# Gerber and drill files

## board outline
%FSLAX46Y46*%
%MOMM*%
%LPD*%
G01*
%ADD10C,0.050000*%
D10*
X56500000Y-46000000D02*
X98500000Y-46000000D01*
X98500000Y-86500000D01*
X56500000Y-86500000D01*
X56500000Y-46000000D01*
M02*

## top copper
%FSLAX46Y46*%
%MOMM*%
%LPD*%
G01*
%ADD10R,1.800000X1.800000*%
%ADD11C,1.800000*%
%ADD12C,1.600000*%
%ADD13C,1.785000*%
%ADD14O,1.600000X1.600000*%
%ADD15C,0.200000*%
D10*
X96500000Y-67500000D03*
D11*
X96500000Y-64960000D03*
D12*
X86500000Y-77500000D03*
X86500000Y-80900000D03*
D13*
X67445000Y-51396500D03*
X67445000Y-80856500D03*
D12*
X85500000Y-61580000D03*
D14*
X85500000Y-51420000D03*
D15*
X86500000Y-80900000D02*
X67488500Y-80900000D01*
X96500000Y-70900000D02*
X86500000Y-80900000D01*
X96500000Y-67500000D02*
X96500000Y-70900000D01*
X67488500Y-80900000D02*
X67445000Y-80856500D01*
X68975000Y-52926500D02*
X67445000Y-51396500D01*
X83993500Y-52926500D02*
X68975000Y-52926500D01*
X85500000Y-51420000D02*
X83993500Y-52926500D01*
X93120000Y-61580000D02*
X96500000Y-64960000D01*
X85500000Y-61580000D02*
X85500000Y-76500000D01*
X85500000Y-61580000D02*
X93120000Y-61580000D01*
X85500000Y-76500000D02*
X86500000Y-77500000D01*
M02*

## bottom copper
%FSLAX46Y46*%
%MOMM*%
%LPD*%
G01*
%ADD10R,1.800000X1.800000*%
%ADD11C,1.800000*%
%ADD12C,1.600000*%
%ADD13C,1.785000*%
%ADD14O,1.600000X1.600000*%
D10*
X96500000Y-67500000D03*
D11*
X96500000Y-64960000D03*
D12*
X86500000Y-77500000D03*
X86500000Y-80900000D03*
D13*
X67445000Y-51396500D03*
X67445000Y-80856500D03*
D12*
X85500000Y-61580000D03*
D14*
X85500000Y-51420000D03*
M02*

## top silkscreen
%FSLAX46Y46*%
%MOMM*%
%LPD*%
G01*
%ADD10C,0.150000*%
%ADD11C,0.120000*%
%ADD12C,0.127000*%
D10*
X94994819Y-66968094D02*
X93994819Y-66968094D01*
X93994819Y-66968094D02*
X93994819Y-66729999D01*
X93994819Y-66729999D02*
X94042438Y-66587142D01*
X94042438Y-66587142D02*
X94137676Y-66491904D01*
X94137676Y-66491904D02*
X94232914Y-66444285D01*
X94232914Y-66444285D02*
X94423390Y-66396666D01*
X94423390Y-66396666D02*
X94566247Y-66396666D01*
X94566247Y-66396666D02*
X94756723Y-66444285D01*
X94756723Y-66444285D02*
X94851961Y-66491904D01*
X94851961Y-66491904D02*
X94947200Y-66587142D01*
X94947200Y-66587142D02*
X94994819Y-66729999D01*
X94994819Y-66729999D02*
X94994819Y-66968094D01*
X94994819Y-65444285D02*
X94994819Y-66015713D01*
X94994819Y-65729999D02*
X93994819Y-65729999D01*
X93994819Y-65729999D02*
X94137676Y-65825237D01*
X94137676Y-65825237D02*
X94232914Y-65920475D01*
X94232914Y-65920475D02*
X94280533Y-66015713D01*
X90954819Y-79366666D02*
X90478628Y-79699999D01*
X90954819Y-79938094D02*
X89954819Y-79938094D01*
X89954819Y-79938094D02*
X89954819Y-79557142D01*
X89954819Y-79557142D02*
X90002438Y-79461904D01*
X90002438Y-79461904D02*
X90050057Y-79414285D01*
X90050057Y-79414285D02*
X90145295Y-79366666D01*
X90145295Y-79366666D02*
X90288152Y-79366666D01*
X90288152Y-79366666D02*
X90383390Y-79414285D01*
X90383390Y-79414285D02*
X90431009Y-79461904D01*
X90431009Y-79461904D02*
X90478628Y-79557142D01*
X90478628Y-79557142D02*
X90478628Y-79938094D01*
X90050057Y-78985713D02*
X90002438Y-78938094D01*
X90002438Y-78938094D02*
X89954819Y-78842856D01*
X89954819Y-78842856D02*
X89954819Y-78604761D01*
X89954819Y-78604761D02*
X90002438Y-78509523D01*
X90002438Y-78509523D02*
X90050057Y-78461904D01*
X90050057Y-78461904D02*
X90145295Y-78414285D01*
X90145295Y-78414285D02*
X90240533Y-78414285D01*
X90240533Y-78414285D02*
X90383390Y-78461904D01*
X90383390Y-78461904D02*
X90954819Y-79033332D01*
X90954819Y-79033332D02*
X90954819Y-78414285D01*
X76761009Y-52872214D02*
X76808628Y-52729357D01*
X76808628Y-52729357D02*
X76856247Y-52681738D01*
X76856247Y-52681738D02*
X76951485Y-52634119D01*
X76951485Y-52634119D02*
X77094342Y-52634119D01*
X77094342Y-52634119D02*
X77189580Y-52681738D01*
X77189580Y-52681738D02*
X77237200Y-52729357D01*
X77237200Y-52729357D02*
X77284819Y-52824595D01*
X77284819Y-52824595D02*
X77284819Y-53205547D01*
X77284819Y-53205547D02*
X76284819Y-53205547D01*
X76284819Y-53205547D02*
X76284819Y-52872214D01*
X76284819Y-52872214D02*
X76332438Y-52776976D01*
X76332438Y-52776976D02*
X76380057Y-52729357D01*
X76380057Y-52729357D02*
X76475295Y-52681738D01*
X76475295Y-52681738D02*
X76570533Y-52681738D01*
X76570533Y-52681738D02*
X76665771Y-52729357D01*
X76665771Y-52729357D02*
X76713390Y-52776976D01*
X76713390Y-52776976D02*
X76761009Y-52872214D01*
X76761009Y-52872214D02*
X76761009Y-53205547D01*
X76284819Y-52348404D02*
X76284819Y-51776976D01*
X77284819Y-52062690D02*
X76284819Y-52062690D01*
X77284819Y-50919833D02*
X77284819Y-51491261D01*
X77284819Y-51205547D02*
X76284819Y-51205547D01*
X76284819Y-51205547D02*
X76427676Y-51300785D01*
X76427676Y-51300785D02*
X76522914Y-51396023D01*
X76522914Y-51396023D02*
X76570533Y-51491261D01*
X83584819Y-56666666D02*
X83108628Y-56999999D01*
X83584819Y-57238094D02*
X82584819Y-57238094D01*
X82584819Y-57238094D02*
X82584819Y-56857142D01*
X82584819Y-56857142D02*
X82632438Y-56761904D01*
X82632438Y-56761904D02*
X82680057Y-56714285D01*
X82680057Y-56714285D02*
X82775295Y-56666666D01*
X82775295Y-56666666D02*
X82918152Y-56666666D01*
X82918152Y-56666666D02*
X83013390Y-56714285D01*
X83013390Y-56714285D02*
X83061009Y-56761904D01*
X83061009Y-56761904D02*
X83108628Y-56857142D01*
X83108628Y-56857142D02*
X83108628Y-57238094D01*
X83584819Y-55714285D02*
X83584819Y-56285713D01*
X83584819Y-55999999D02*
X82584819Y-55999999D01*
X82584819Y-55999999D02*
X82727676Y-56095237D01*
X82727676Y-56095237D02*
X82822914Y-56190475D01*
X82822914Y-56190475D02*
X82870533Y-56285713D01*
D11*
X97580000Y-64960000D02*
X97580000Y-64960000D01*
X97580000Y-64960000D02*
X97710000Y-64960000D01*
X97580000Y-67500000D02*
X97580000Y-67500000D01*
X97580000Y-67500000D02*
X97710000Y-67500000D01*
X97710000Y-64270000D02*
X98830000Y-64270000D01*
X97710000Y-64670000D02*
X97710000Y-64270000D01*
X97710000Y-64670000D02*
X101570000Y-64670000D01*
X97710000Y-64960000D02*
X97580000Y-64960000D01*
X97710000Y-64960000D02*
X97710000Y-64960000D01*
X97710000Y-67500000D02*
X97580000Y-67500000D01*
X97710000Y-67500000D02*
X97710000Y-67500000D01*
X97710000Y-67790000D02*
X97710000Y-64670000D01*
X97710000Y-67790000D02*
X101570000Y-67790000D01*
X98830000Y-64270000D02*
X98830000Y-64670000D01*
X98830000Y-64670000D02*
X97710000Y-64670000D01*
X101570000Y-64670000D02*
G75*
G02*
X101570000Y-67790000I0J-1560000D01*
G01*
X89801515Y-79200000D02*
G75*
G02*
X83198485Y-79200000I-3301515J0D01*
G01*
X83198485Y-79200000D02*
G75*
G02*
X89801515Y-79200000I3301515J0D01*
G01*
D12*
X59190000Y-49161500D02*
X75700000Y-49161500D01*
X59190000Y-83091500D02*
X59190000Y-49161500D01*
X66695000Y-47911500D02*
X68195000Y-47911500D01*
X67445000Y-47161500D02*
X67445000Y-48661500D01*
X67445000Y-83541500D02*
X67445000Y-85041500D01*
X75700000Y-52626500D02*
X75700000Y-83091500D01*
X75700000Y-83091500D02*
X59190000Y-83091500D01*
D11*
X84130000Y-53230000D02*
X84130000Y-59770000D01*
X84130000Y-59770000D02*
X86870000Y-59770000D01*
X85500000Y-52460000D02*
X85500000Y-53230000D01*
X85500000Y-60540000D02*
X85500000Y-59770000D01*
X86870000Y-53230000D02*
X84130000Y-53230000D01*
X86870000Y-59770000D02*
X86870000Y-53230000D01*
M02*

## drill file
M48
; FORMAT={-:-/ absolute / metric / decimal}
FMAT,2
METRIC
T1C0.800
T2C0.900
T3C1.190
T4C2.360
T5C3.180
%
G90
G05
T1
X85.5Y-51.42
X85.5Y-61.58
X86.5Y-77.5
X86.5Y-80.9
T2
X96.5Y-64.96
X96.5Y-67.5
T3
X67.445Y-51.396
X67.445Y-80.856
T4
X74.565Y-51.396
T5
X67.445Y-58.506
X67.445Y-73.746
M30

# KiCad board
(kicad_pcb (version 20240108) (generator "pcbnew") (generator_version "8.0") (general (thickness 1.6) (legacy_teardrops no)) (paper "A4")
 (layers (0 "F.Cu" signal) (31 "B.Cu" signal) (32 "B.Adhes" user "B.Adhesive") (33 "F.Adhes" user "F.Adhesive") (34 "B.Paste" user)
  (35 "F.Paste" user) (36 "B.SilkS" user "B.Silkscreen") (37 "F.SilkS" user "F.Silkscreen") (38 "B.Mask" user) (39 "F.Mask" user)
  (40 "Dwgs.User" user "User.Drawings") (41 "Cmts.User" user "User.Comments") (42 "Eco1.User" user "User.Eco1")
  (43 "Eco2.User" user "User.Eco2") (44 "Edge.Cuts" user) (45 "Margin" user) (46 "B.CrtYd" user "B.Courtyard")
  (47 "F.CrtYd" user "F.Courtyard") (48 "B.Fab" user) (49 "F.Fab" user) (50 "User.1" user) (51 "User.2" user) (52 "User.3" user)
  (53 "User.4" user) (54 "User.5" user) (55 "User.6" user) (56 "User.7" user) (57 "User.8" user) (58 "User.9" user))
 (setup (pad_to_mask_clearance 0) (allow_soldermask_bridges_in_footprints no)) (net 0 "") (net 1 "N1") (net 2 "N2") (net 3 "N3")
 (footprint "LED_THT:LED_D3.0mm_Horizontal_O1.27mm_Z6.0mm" (layer "F.Cu") (at 96.5 67.5 90)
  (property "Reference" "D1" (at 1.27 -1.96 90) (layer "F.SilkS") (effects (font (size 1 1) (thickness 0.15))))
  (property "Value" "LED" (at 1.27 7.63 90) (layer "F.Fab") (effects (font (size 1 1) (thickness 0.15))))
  (fp_line (start 2.54 1.08) (end 2.54 1.08) (stroke (width 0.12) (type solid)) (layer "F.SilkS"))
  (fp_line (start 2.54 1.08) (end 2.54 1.21) (stroke (width 0.12) (type solid)) (layer "F.SilkS"))
  (fp_line (start 0 1.08) (end 0 1.08) (stroke (width 0.12) (type solid)) (layer "F.SilkS"))
  (fp_line (start 0 1.08) (end 0 1.21) (stroke (width 0.12) (type solid)) (layer "F.SilkS"))
  (fp_line (start 3.23 1.21) (end 3.23 2.33) (stroke (width 0.12) (type solid)) (layer "F.SilkS"))
  (fp_line (start 2.83 1.21) (end 3.23 1.21) (stroke (width 0.12) (type solid)) (layer "F.SilkS"))
  (fp_line (start 2.83 1.21) (end 2.83 5.07) (stroke (width 0.12) (type solid)) (layer "F.SilkS"))
  (fp_line (start 2.54 1.21) (end 2.54 1.08) (stroke (width 0.12) (type solid)) (layer "F.SilkS"))
  (fp_line (start 2.54 1.21) (end 2.54 1.21) (stroke (width 0.12) (type solid)) (layer "F.SilkS"))
  (fp_line (start 0 1.21) (end 0 1.08) (stroke (width 0.12) (type solid)) (layer "F.SilkS"))
  (fp_line (start 0 1.21) (end 0 1.21) (stroke (width 0.12) (type solid)) (layer "F.SilkS"))
  (fp_line (start -0.29 1.21) (end 2.83 1.21) (stroke (width 0.12) (type solid)) (layer "F.SilkS"))
  (fp_line (start -0.29 1.21) (end -0.29 5.07) (stroke (width 0.12) (type solid)) (layer "F.SilkS"))
  (fp_line (start 3.23 2.33) (end 2.83 2.33) (stroke (width 0.12) (type solid)) (layer "F.SilkS"))
  (fp_line (start 2.83 2.33) (end 2.83 1.21) (stroke (width 0.12) (type solid)) (layer "F.SilkS"))
  (fp_arc (start 2.83 5.07) (mid 1.27 6.63) (end -0.29 5.07) (stroke (width 0.12) (type solid)) (layer "F.SilkS"))
  (pad "1" thru_hole rect (at 0 0 90) (size 1.8 1.8) (drill 0.9) (layers "*.Cu" "*.Mask") (remove_unused_layers no) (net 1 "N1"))
  (pad "2" thru_hole circle (at 2.54 0 90) (size 1.8 1.8) (drill 0.9) (layers "*.Cu" "*.Mask") (remove_unused_layers no) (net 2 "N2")))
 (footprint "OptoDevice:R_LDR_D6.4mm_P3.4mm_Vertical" (layer "F.Cu") (at 86.5 77.5 -90)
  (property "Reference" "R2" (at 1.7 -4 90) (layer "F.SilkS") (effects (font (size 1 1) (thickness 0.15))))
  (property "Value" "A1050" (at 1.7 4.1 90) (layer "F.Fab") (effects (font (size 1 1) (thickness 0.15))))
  (fp_circle (center 1.7 0) (end 5 -0.1) (stroke (width 0.12) (type solid)) (fill none) (layer "F.SilkS"))
  (pad "1" thru_hole circle (at 0 0 270) (size 1.6 1.6) (drill 0.8) (layers "*.Cu" "*.Mask") (remove_unused_layers no) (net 2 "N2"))
  (pad "2" thru_hole circle (at 3.4 0 270) (size 1.6 1.6) (drill 0.8) (layers "*.Cu" "*.Mask") (remove_unused_layers no) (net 1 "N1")))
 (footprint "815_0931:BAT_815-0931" (layer "F.Cu") (at 67.445 66.1265 -90)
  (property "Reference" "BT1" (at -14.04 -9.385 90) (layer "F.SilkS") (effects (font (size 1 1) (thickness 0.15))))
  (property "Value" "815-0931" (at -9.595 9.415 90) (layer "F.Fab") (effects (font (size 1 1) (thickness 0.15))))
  (fp_line (start -16.965 8.255) (end -16.965 -8.255) (stroke (width 0.127) (type solid)) (layer "F.SilkS"))
  (fp_line (start 16.965 8.255) (end -16.965 8.255) (stroke (width 0.127) (type solid)) (layer "F.SilkS"))
  (fp_line (start -18.215 0.75) (end -18.215 -0.75) (stroke (width 0.127) (type solid)) (layer "F.SilkS"))
  (fp_line (start -18.965 0) (end -17.465 0) (stroke (width 0.127) (type solid)) (layer "F.SilkS"))
  (fp_line (start 17.415 0) (end 18.915 0) (stroke (width 0.127) (type solid)) (layer "F.SilkS"))
  (fp_line (start -13.5 -8.255) (end 16.965 -8.255) (stroke (width 0.127) (type solid)) (layer "F.SilkS"))
  (fp_line (start 16.965 -8.255) (end 16.965 8.255) (stroke (width 0.127) (type solid)) (layer "F.SilkS"))
  (pad "" np_thru_hole circle (at -14.73 -7.12 270) (size 2.36 2.36) (drill 2.36) (layers "*.Cu" "*.Mask"))
  (pad "" np_thru_hole circle (at -7.62 0 270) (size 3.18 3.18) (drill 3.18) (layers "*.Cu" "*.Mask"))
  (pad "" np_thru_hole circle (at 7.62 0 270) (size 3.18 3.18) (drill 3.18) (layers "*.Cu" "*.Mask"))
  (pad "+" thru_hole circle (at -14.73 0 270) (size 1.785 1.785) (drill 1.19) (layers "*.Cu" "*.Mask") (remove_unused_layers no)
   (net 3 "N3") (solder_mask_margin 0.102))
  (pad "-" thru_hole circle (at 14.73 0 270) (size 1.785 1.785) (drill 1.19) (layers "*.Cu" "*.Mask") (remove_unused_layers no) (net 1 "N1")
   (solder_mask_margin 0.102)))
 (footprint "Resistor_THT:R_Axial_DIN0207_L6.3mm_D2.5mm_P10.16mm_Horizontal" (layer "F.Cu") (at 85.5 61.58 90)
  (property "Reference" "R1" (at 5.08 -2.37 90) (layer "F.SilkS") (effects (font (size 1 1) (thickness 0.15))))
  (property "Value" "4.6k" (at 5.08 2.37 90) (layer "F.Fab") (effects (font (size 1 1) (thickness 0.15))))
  (fp_line (start 8.35 -1.37) (end 1.81 -1.37) (stroke (width 0.12) (type solid)) (layer "F.SilkS"))
  (fp_line (start 1.81 -1.37) (end 1.81 1.37) (stroke (width 0.12) (type solid)) (layer "F.SilkS"))
  (fp_line (start 9.12 0) (end 8.35 0) (stroke (width 0.12) (type solid)) (layer "F.SilkS"))
  (fp_line (start 1.04 0) (end 1.81 0) (stroke (width 0.12) (type solid)) (layer "F.SilkS"))
  (fp_line (start 8.35 1.37) (end 8.35 -1.37) (stroke (width 0.12) (type solid)) (layer "F.SilkS"))
  (fp_line (start 1.81 1.37) (end 8.35 1.37) (stroke (width 0.12) (type solid)) (layer "F.SilkS"))
  (pad "1" thru_hole circle (at 0 0 90) (size 1.6 1.6) (drill 0.8) (layers "*.Cu" "*.Mask") (remove_unused_layers no) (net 2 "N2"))
  (pad "2" thru_hole oval (at 10.16 0 90) (size 1.6 1.6) (drill 0.8) (layers "*.Cu" "*.Mask") (remove_unused_layers no) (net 3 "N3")))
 (gr_rect (start 56.5 46) (end 98.5 86.5) (stroke (width 0.05) (type default)) (fill none) (layer "Edge.Cuts"))
 (segment (start 86.5 80.9) (end 67.4885 80.9) (width 0.2) (layer "F.Cu") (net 1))
 (segment (start 96.5 70.9) (end 86.5 80.9) (width 0.2) (layer "F.Cu") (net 1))
 (segment (start 96.5 67.5) (end 96.5 70.9) (width 0.2) (layer "F.Cu") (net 1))
 (segment (start 67.4885 80.9) (end 67.445 80.8565) (width 0.2) (layer "F.Cu") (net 1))
 (segment (start 68.975 52.9265) (end 67.445 51.3965) (width 0.2) (layer "F.Cu") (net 3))
 (segment (start 83.9935 52.9265) (end 68.975 52.9265) (width 0.2) (layer "F.Cu") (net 3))
 (segment (start 85.5 51.42) (end 83.9935 52.9265) (width 0.2) (layer "F.Cu") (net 3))
 (segment (start 93.12 61.58) (end 96.5 64.96) (width 0.2) (layer "F.Cu") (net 2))
 (segment (start 85.5 61.58) (end 85.5 76.5) (width 0.2) (layer "F.Cu") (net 2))
 (segment (start 85.5 61.58) (end 93.12 61.58) (width 0.2) (layer "F.Cu") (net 2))
 (segment (start 85.5 76.5) (end 86.5 77.5) (width 0.2) (layer "F.Cu") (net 2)))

